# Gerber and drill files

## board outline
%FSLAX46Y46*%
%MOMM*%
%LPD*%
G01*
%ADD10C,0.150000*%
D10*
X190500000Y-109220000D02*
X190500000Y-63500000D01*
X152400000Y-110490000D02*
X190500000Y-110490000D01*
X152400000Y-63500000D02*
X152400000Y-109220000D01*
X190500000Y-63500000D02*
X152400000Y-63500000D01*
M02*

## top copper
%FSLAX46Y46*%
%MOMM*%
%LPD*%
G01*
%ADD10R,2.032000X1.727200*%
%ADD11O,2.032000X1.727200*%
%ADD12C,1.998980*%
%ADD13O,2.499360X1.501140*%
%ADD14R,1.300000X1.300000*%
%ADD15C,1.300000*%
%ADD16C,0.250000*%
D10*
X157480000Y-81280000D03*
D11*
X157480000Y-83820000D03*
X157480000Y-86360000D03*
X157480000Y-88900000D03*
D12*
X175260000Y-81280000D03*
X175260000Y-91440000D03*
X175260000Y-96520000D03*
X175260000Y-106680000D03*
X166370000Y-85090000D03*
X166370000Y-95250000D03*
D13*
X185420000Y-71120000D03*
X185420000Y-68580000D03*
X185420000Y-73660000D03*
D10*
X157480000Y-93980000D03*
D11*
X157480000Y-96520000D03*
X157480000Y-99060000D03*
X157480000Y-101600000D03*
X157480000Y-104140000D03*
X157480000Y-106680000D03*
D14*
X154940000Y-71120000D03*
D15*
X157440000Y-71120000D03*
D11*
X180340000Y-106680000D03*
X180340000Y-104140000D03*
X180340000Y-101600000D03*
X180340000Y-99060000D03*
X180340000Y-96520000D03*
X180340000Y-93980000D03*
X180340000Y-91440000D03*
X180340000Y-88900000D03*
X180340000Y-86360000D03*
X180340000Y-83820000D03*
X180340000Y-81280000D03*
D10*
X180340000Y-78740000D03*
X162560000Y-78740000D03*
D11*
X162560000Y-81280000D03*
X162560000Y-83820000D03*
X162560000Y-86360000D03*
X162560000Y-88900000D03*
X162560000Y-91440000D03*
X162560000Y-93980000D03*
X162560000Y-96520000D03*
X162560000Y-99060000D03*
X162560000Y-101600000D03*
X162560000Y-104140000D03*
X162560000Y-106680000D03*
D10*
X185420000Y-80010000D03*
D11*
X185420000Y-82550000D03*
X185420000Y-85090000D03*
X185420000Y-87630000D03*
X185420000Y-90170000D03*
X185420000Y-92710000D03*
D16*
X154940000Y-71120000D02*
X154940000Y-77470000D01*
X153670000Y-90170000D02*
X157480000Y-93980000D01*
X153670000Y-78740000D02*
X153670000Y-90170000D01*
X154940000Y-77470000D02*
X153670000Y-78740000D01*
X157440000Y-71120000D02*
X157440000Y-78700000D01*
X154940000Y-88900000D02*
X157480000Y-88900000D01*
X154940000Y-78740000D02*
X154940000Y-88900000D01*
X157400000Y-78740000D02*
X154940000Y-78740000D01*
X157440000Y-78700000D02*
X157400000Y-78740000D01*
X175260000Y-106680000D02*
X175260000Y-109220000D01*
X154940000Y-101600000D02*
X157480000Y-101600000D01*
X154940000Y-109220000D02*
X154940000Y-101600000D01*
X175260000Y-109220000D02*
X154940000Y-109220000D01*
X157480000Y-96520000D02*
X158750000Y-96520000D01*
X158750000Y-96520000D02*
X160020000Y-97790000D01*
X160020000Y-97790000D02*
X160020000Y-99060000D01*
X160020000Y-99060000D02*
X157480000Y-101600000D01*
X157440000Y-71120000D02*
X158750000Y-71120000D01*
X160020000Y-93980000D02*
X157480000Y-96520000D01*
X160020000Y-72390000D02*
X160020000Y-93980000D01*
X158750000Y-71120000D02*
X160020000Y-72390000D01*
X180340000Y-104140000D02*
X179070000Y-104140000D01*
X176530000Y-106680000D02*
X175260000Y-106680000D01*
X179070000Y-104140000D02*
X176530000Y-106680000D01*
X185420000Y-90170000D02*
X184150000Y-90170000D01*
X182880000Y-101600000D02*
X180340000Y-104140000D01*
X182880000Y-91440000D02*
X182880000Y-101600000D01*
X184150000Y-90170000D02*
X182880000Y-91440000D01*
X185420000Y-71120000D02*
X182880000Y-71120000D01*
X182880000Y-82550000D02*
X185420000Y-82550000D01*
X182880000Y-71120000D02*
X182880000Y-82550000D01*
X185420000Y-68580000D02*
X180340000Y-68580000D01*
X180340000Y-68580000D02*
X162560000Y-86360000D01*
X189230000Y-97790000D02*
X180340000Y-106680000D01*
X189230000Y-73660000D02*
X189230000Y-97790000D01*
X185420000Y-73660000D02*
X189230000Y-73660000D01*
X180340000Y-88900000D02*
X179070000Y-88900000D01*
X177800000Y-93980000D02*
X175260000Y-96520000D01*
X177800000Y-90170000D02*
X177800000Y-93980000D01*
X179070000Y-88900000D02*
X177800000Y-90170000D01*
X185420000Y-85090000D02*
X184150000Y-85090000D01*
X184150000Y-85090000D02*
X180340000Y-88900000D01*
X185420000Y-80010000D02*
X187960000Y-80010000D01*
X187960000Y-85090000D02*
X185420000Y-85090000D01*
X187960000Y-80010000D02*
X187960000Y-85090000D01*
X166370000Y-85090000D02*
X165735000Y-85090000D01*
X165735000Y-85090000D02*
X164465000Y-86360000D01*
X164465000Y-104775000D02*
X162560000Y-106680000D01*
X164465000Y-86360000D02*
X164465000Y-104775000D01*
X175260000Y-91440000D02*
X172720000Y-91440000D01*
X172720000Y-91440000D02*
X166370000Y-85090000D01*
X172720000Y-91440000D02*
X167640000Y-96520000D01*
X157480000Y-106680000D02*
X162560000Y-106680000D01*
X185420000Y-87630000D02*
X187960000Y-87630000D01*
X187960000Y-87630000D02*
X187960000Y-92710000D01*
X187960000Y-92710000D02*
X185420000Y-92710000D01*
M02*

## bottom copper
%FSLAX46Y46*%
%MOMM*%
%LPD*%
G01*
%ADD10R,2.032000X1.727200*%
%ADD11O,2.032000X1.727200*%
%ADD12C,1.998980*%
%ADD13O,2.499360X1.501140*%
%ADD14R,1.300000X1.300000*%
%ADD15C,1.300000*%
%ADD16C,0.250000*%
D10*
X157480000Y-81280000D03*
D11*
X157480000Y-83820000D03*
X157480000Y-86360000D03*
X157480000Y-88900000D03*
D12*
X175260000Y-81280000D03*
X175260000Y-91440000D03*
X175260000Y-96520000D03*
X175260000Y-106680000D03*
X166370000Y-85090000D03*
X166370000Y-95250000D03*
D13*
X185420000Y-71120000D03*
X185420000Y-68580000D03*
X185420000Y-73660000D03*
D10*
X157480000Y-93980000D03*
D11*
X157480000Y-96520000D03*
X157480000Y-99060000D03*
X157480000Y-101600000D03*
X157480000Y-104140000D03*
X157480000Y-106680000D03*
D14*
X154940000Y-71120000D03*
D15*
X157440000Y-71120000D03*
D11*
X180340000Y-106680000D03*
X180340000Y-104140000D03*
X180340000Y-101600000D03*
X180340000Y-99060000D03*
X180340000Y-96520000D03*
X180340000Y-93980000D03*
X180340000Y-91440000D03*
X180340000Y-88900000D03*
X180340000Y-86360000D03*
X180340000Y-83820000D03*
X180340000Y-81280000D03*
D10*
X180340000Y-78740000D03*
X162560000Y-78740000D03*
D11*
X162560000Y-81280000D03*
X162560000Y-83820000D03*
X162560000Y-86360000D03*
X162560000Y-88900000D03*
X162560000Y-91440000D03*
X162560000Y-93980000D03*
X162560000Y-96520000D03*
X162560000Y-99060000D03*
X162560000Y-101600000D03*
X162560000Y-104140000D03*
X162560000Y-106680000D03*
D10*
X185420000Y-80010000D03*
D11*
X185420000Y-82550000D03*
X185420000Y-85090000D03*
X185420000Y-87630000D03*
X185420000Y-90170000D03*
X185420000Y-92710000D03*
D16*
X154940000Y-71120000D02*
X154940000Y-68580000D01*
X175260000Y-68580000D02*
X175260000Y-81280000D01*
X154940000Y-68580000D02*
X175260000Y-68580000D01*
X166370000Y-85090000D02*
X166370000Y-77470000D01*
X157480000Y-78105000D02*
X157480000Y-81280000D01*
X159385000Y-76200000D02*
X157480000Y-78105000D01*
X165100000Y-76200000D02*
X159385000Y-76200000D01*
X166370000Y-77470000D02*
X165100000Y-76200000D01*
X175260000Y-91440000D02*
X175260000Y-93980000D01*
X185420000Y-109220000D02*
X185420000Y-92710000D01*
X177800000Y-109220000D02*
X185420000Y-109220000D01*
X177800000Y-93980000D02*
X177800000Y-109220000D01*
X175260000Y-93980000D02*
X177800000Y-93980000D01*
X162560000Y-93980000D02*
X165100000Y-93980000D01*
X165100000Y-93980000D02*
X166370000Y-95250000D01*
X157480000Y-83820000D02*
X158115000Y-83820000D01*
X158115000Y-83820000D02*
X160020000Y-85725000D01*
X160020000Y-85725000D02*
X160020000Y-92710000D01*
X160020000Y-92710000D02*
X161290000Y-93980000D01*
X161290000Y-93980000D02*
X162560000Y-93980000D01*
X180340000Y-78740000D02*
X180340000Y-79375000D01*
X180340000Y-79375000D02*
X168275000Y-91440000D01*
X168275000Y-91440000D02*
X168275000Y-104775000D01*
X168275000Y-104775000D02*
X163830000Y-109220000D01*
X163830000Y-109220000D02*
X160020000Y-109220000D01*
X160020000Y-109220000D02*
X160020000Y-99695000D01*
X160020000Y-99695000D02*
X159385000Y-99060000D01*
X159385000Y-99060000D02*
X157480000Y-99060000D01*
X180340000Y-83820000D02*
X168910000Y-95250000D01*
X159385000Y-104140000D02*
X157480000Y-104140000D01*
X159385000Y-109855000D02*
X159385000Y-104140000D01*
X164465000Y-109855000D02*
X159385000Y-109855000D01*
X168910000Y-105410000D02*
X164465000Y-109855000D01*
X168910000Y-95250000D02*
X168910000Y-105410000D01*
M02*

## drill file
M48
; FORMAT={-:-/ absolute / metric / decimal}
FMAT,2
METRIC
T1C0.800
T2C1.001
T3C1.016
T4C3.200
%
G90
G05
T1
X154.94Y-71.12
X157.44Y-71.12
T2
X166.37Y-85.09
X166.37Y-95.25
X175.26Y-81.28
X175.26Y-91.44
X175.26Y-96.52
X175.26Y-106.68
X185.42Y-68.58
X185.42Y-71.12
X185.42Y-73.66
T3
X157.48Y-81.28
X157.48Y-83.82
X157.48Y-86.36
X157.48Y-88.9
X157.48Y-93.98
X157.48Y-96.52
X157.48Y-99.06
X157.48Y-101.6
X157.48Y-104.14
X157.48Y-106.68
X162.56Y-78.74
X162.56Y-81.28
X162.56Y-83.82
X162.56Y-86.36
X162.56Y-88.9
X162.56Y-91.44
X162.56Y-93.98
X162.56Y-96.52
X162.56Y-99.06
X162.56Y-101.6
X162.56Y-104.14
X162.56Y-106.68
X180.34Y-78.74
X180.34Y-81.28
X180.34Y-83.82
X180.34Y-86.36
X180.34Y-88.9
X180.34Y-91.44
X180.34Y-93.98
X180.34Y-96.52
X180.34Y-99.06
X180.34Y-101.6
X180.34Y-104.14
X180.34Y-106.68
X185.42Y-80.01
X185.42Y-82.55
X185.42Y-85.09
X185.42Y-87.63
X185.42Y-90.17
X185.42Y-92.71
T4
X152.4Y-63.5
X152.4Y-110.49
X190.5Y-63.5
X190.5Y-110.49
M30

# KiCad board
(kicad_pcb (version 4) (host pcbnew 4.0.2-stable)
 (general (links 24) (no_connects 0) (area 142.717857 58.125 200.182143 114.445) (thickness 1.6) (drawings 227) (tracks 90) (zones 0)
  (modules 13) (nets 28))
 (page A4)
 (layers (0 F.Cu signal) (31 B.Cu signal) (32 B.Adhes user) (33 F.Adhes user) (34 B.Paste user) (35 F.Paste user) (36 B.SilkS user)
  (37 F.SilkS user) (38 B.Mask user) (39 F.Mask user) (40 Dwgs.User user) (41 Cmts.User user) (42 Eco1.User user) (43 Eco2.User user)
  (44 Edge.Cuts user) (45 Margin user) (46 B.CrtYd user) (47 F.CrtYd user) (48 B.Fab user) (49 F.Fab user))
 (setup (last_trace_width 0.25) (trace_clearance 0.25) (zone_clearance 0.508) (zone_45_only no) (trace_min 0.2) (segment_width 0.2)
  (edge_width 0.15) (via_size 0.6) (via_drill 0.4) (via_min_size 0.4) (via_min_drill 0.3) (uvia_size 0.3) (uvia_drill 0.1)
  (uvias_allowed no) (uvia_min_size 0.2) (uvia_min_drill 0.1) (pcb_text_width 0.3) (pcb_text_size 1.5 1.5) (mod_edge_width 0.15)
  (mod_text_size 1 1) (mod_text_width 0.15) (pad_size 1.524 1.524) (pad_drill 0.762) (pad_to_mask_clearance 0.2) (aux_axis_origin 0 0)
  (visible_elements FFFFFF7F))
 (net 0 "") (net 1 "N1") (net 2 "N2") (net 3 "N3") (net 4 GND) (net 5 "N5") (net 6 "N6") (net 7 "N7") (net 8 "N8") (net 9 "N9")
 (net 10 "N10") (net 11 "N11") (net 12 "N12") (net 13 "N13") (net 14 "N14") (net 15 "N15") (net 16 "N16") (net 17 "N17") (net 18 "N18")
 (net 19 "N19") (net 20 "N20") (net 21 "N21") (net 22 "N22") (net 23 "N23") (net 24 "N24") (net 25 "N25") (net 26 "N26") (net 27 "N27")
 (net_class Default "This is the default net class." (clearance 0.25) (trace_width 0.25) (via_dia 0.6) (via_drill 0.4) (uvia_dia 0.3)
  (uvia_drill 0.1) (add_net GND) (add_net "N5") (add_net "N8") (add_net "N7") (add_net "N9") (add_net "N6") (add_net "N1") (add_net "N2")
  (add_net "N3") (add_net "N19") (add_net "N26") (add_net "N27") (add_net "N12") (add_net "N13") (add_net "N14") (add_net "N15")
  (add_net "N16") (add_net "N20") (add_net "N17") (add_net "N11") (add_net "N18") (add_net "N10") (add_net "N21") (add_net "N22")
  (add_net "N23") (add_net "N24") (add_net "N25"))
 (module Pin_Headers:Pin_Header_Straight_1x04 (layer F.Cu) (at 157.48 81.28)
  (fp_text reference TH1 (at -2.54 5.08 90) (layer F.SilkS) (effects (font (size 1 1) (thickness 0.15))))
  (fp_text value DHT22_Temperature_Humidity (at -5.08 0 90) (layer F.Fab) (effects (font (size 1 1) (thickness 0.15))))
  (pad 1 thru_hole rect (at 0 0) (size 2.032 1.7272) (drill 1.016) (layers *.Cu *.Mask F.SilkS) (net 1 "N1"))
  (pad 2 thru_hole oval (at 0 2.54) (size 2.032 1.7272) (drill 1.016) (layers *.Cu *.Mask F.SilkS) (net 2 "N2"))
  (pad 3 thru_hole oval (at 0 5.08) (size 2.032 1.7272) (drill 1.016) (layers *.Cu *.Mask F.SilkS) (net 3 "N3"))
  (pad 4 thru_hole oval (at 0 7.62) (size 2.032 1.7272) (drill 1.016) (layers *.Cu *.Mask F.SilkS) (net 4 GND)))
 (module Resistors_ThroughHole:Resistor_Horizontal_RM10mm (layer F.Cu) (at 175.26 81.28 270)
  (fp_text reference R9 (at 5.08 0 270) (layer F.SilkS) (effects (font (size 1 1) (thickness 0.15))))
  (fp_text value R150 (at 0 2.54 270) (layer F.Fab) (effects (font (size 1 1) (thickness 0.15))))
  (pad 1 thru_hole circle (at 0 0 270) (size 1.99898 1.99898) (drill 1.00076) (layers *.Cu *.SilkS *.Mask) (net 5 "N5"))
  (pad 2 thru_hole circle (at 10.16 0 270) (size 1.99898 1.99898) (drill 1.00076) (layers *.Cu *.SilkS *.Mask) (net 1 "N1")))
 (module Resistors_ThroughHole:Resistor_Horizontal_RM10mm (layer F.Cu) (at 175.26 96.52 270)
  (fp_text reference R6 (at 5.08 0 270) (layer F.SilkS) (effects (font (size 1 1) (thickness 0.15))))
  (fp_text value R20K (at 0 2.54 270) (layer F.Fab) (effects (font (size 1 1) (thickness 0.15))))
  (pad 1 thru_hole circle (at 0 0 270) (size 1.99898 1.99898) (drill 1.00076) (layers *.Cu *.SilkS *.Mask) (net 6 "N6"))
  (pad 2 thru_hole circle (at 10.16 0 270) (size 1.99898 1.99898) (drill 1.00076) (layers *.Cu *.SilkS *.Mask) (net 4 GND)))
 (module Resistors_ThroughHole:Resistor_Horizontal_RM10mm (layer F.Cu) (at 166.37 85.09 270)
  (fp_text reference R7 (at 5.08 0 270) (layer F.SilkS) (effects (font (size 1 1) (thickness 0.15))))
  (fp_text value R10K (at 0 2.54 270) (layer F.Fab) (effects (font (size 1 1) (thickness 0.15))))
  (pad 1 thru_hole circle (at 0 0 270) (size 1.99898 1.99898) (drill 1.00076) (layers *.Cu *.SilkS *.Mask) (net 1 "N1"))
  (pad 2 thru_hole circle (at 10.16 0 270) (size 1.99898 1.99898) (drill 1.00076) (layers *.Cu *.SilkS *.Mask) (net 2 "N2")))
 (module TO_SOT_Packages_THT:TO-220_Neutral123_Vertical (layer F.Cu) (at 185.42 71.12 270)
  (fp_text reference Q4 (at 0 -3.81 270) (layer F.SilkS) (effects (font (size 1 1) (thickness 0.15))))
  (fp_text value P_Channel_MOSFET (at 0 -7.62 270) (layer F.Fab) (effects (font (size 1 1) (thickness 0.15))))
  (pad 2 thru_hole oval (at 0 0) (size 2.49936 1.50114) (drill 1.00076) (layers *.Cu *.Mask F.SilkS) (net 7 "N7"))
  (pad 1 thru_hole oval (at -2.54 0) (size 2.49936 1.50114) (drill 1.00076) (layers *.Cu *.Mask F.SilkS) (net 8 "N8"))
  (pad 3 thru_hole oval (at 2.54 0) (size 2.49936 1.50114) (drill 1.00076) (layers *.Cu *.Mask F.SilkS) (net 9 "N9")))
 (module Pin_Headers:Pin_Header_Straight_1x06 (layer F.Cu) (at 157.48 93.98)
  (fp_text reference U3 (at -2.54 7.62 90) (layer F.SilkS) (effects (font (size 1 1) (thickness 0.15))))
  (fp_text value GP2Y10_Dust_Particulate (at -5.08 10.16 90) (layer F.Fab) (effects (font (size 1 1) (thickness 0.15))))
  (pad 1 thru_hole rect (at 0 0) (size 2.032 1.7272) (drill 1.016) (layers *.Cu *.Mask F.SilkS) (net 5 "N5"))
  (pad 2 thru_hole oval (at 0 2.54) (size 2.032 1.7272) (drill 1.016) (layers *.Cu *.Mask F.SilkS) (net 4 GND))
  (pad 3 thru_hole oval (at 0 5.08) (size 2.032 1.7272) (drill 1.016) (layers *.Cu *.Mask F.SilkS) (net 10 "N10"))
  (pad 4 thru_hole oval (at 0 7.62) (size 2.032 1.7272) (drill 1.016) (layers *.Cu *.Mask F.SilkS) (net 4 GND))
  (pad 5 thru_hole oval (at 0 10.16) (size 2.032 1.7272) (drill 1.016) (layers *.Cu *.Mask F.SilkS) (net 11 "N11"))
  (pad 6 thru_hole oval (at 0 12.7) (size 2.032 1.7272) (drill 1.016) (layers *.Cu *.Mask F.SilkS) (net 1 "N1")))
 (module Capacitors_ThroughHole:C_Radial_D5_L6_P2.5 (layer F.Cu) (at 154.94 71.12)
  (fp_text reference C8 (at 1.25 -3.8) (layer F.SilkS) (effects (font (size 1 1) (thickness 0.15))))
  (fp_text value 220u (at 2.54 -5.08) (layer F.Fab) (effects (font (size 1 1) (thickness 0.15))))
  (pad 1 thru_hole rect (at 0 0) (size 1.3 1.3) (drill 0.8) (layers *.Cu *.Mask F.SilkS) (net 5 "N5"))
  (pad 2 thru_hole circle (at 2.5 0) (size 1.3 1.3) (drill 0.8) (layers *.Cu *.Mask F.SilkS) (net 4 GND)))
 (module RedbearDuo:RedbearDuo (layer F.Cu) (at 162.56 78.74)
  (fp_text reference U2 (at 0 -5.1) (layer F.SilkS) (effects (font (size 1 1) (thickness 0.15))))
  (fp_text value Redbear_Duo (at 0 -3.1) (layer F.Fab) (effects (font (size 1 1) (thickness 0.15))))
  (pad 13 thru_hole oval (at 17.78 27.94) (size 2.032 1.7272) (drill 1.016) (layers *.Cu *.Mask F.SilkS) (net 9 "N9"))
  (pad 14 thru_hole oval (at 17.78 25.4) (size 2.032 1.7272) (drill 1.016) (layers *.Cu *.Mask F.SilkS) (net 4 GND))
  (pad 15 thru_hole oval (at 17.78 22.86) (size 2.032 1.7272) (drill 1.016) (layers *.Cu *.Mask F.SilkS) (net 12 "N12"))
  (pad 16 thru_hole oval (at 17.78 20.32) (size 2.032 1.7272) (drill 1.016) (layers *.Cu *.Mask F.SilkS) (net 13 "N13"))
  (pad 17 thru_hole oval (at 17.78 17.78) (size 2.032 1.7272) (drill 1.016) (layers *.Cu *.Mask F.SilkS) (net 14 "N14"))
  (pad 18 thru_hole oval (at 17.78 15.24) (size 2.032 1.7272) (drill 1.016) (layers *.Cu *.Mask F.SilkS) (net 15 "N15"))
  (pad 19 thru_hole oval (at 17.78 12.7) (size 2.032 1.7272) (drill 1.016) (layers *.Cu *.Mask F.SilkS) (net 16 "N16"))
  (pad 20 thru_hole oval (at 17.78 10.16) (size 2.032 1.7272) (drill 1.016) (layers *.Cu *.Mask F.SilkS) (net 6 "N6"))
  (pad 21 thru_hole oval (at 17.78 7.62) (size 2.032 1.7272) (drill 1.016) (layers *.Cu *.Mask F.SilkS) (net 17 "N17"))
  (pad 22 thru_hole oval (at 17.78 5.08) (size 2.032 1.7272) (drill 1.016) (layers *.Cu *.Mask F.SilkS) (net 11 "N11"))
  (pad 23 thru_hole oval (at 17.78 2.54) (size 2.032 1.7272) (drill 1.016) (layers *.Cu *.Mask F.SilkS) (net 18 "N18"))
  (pad 24 thru_hole rect (at 17.78 0) (size 2.032 1.7272) (drill 1.016) (layers *.Cu *.Mask F.SilkS) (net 10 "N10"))
  (pad 1 thru_hole rect (at 0 0) (size 2.032 1.7272) (drill 1.016) (layers *.Cu *.Mask F.SilkS) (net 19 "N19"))
  (pad 2 thru_hole oval (at 0 2.54) (size 2.032 1.7272) (drill 1.016) (layers *.Cu *.Mask F.SilkS) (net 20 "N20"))
  (pad 3 thru_hole oval (at 0 5.08) (size 2.032 1.7272) (drill 1.016) (layers *.Cu *.Mask F.SilkS) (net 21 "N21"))
  (pad 4 thru_hole oval (at 0 7.62) (size 2.032 1.7272) (drill 1.016) (layers *.Cu *.Mask F.SilkS) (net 8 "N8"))
  (pad 5 thru_hole oval (at 0 10.16) (size 2.032 1.7272) (drill 1.016) (layers *.Cu *.Mask F.SilkS) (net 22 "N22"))
  (pad 6 thru_hole oval (at 0 12.7) (size 2.032 1.7272) (drill 1.016) (layers *.Cu *.Mask F.SilkS) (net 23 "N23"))
  (pad 7 thru_hole oval (at 0 15.24) (size 2.032 1.7272) (drill 1.016) (layers *.Cu *.Mask F.SilkS) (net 2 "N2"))
  (pad 8 thru_hole oval (at 0 17.78) (size 2.032 1.7272) (drill 1.016) (layers *.Cu *.Mask F.SilkS) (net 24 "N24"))
  (pad 9 thru_hole oval (at 0 20.32) (size 2.032 1.7272) (drill 1.016) (layers *.Cu *.Mask F.SilkS) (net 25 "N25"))
  (pad 10 thru_hole oval (at 0 22.86) (size 2.032 1.7272) (drill 1.016) (layers *.Cu *.Mask F.SilkS) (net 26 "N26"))
  (pad 11 thru_hole oval (at 0 25.4) (size 2.032 1.7272) (drill 1.016) (layers *.Cu *.Mask F.SilkS) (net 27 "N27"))
  (pad 12 thru_hole oval (at 0 27.94) (size 2.032 1.7272) (drill 1.016) (layers *.Cu *.Mask F.SilkS) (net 1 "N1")))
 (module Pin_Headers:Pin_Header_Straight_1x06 (layer F.Cu) (at 185.42 80.01)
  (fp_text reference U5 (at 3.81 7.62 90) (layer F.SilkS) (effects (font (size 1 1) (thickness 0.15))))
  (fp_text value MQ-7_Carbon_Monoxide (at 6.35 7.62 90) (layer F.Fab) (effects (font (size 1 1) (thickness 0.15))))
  (pad 1 thru_hole rect (at 0 0) (size 2.032 1.7272) (drill 1.016) (layers *.Cu *.Mask F.SilkS) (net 6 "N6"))
  (pad 2 thru_hole oval (at 0 2.54) (size 2.032 1.7272) (drill 1.016) (layers *.Cu *.Mask F.SilkS) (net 7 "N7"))
  (pad 3 thru_hole oval (at 0 5.08) (size 2.032 1.7272) (drill 1.016) (layers *.Cu *.Mask F.SilkS) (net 6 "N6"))
  (pad 4 thru_hole oval (at 0 7.62) (size 2.032 1.7272) (drill 1.016) (layers *.Cu *.Mask F.SilkS) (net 1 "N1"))
  (pad 5 thru_hole oval (at 0 10.16) (size 2.032 1.7272) (drill 1.016) (layers *.Cu *.Mask F.SilkS) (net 4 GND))
  (pad 6 thru_hole oval (at 0 12.7) (size 2.032 1.7272) (drill 1.016) (layers *.Cu *.Mask F.SilkS) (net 1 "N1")))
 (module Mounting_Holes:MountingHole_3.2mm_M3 (layer F.Cu) (at 190.5 63.5)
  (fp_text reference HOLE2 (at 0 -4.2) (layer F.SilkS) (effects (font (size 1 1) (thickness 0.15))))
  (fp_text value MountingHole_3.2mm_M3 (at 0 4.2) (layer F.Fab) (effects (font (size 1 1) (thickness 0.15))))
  (pad 1 np_thru_hole circle (at 0 0) (size 3.2 3.2) (drill 3.2) (layers *.Cu *.Mask F.SilkS)))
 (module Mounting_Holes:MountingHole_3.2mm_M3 (layer F.Cu) (at 190.5 110.49)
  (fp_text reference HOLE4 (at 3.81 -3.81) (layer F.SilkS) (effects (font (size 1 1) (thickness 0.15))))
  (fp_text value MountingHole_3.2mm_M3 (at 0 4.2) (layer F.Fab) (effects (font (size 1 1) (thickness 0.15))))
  (pad 1 np_thru_hole circle (at 0 0) (size 3.2 3.2) (drill 3.2) (layers *.Cu *.Mask F.SilkS)))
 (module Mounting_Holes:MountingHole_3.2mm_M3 (layer F.Cu) (at 152.4 63.5)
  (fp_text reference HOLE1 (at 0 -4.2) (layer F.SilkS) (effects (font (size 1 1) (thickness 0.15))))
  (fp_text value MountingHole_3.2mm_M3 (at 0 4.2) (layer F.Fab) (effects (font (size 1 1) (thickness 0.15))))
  (pad 1 np_thru_hole circle (at 0 0) (size 3.2 3.2) (drill 3.2) (layers *.Cu *.Mask F.SilkS)))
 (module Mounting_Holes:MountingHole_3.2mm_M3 (layer F.Cu) (at 152.4 110.49)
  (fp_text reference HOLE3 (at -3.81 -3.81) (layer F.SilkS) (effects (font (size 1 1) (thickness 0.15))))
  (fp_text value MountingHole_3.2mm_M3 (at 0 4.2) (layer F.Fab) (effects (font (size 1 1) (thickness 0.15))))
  (pad 1 np_thru_hole circle (at 0 0) (size 3.2 3.2) (drill 3.2) (layers *.Cu *.Mask F.SilkS)))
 (gr_line (start 190.5 109.22) (end 190.5 63.5) (angle 90) (layer Edge.Cuts) (width 0.15))
 (gr_line (start 152.4 110.49) (end 190.5 110.49) (angle 90) (layer Edge.Cuts) (width 0.15))
 (gr_line (start 152.4 63.5) (end 152.4 109.22) (angle 90) (layer Edge.Cuts) (width 0.15))
 (gr_line (start 190.5 63.5) (end 152.4 63.5) (angle 90) (layer Edge.Cuts) (width 0.15))
 (segment (start 154.94 71.12) (end 154.94 68.58) (width 0.25) (layer B.Cu) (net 5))
 (segment (start 175.26 68.58) (end 175.26 81.28) (width 0.25) (layer B.Cu) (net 5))
 (segment (start 154.94 68.58) (end 175.26 68.58) (width 0.25) (layer B.Cu) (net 5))
 (segment (start 154.94 71.12) (end 154.94 77.47) (width 0.25) (layer F.Cu) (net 5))
 (segment (start 153.67 90.17) (end 157.48 93.98) (width 0.25) (layer F.Cu) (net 5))
 (segment (start 153.67 78.74) (end 153.67 90.17) (width 0.25) (layer F.Cu) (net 5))
 (segment (start 154.94 77.47) (end 153.67 78.74) (width 0.25) (layer F.Cu) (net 5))
 (segment (start 157.44 71.12) (end 157.44 78.7) (width 0.25) (layer F.Cu) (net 4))
 (segment (start 154.94 88.9) (end 157.48 88.9) (width 0.25) (layer F.Cu) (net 4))
 (segment (start 154.94 78.74) (end 154.94 88.9) (width 0.25) (layer F.Cu) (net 4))
 (segment (start 157.4 78.74) (end 154.94 78.74) (width 0.25) (layer F.Cu) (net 4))
 (segment (start 157.44 78.7) (end 157.4 78.74) (width 0.25) (layer F.Cu) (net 4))
 (segment (start 175.26 106.68) (end 175.26 109.22) (width 0.25) (layer F.Cu) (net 4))
 (segment (start 154.94 101.6) (end 157.48 101.6) (width 0.25) (layer F.Cu) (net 4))
 (segment (start 154.94 109.22) (end 154.94 101.6) (width 0.25) (layer F.Cu) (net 4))
 (segment (start 175.26 109.22) (end 154.94 109.22) (width 0.25) (layer F.Cu) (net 4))
 (segment (start 157.48 96.52) (end 158.75 96.52) (width 0.25) (layer F.Cu) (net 4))
 (segment (start 158.75 96.52) (end 160.02 97.79) (width 0.25) (layer F.Cu) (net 4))
 (segment (start 160.02 97.79) (end 160.02 99.06) (width 0.25) (layer F.Cu) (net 4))
 (segment (start 160.02 99.06) (end 157.48 101.6) (width 0.25) (layer F.Cu) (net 4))
 (segment (start 157.44 71.12) (end 158.75 71.12) (width 0.25) (layer F.Cu) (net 4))
 (segment (start 160.02 93.98) (end 157.48 96.52) (width 0.25) (layer F.Cu) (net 4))
 (segment (start 160.02 72.39) (end 160.02 93.98) (width 0.25) (layer F.Cu) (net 4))
 (segment (start 158.75 71.12) (end 160.02 72.39) (width 0.25) (layer F.Cu) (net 4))
 (segment (start 180.34 104.14) (end 179.07 104.14) (width 0.25) (layer F.Cu) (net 4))
 (segment (start 176.53 106.68) (end 175.26 106.68) (width 0.25) (layer F.Cu) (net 4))
 (segment (start 179.07 104.14) (end 176.53 106.68) (width 0.25) (layer F.Cu) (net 4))
 (segment (start 185.42 90.17) (end 184.15 90.17) (width 0.25) (layer F.Cu) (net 4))
 (segment (start 182.88 101.6) (end 180.34 104.14) (width 0.25) (layer F.Cu) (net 4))
 (segment (start 182.88 91.44) (end 182.88 101.6) (width 0.25) (layer F.Cu) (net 4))
 (segment (start 184.15 90.17) (end 182.88 91.44) (width 0.25) (layer F.Cu) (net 4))
 (segment (start 185.42 71.12) (end 182.88 71.12) (width 0.25) (layer F.Cu) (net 7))
 (segment (start 182.88 82.55) (end 185.42 82.55) (width 0.25) (layer F.Cu) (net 7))
 (segment (start 182.88 71.12) (end 182.88 82.55) (width 0.25) (layer F.Cu) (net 7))
 (segment (start 185.42 68.58) (end 180.34 68.58) (width 0.25) (layer F.Cu) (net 8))
 (segment (start 180.34 68.58) (end 162.56 86.36) (width 0.25) (layer F.Cu) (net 8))
 (segment (start 189.23 97.79) (end 180.34 106.68) (width 0.25) (layer F.Cu) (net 9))
 (segment (start 189.23 73.66) (end 189.23 97.79) (width 0.25) (layer F.Cu) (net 9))
 (segment (start 185.42 73.66) (end 189.23 73.66) (width 0.25) (layer F.Cu) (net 9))
 (segment (start 180.34 88.9) (end 179.07 88.9) (width 0.25) (layer F.Cu) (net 6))
 (segment (start 177.8 93.98) (end 175.26 96.52) (width 0.25) (layer F.Cu) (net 6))
 (segment (start 177.8 90.17) (end 177.8 93.98) (width 0.25) (layer F.Cu) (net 6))
 (segment (start 179.07 88.9) (end 177.8 90.17) (width 0.25) (layer F.Cu) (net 6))
 (segment (start 185.42 85.09) (end 184.15 85.09) (width 0.25) (layer F.Cu) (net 6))
 (segment (start 184.15 85.09) (end 180.34 88.9) (width 0.25) (layer F.Cu) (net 6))
 (segment (start 185.42 80.01) (end 187.96 80.01) (width 0.25) (layer F.Cu) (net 6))
 (segment (start 187.96 85.09) (end 185.42 85.09) (width 0.25) (layer F.Cu) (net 6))
 (segment (start 187.96 80.01) (end 187.96 85.09) (width 0.25) (layer F.Cu) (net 6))
 (segment (start 166.37 85.09) (end 166.37 77.47) (width 0.25) (layer B.Cu) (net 1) (status 400000))
 (segment (start 157.48 78.105) (end 157.48 81.28) (width 0.25) (layer B.Cu) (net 1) (status 800000))
 (segment (start 159.385 76.2) (end 157.48 78.105) (width 0.25) (layer B.Cu) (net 1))
 (segment (start 165.1 76.2) (end 159.385 76.2) (width 0.25) (layer B.Cu) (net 1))
 (segment (start 166.37 77.47) (end 165.1 76.2) (width 0.25) (layer B.Cu) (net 1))
 (segment (start 166.37 85.09) (end 165.735 85.09) (width 0.25) (layer F.Cu) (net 1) (status C00000))
 (segment (start 165.735 85.09) (end 164.465 86.36) (width 0.25) (layer F.Cu) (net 1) (status 400000))
 (segment (start 164.465 104.775) (end 162.56 106.68) (width 0.25) (layer F.Cu) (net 1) (status 800000))
 (segment (start 164.465 86.36) (end 164.465 104.775) (width 0.25) (layer F.Cu) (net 1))
 (segment (start 175.26 91.44) (end 172.72 91.44) (width 0.25) (layer F.Cu) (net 1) (status 400000))
 (segment (start 172.72 91.44) (end 166.37 85.09) (width 0.25) (layer F.Cu) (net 1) (status 800000))
 (segment (start 175.26 91.44) (end 175.26 93.98) (width 0.25) (layer B.Cu) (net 1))
 (segment (start 185.42 109.22) (end 185.42 92.71) (width 0.25) (layer B.Cu) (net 1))
 (segment (start 177.8 109.22) (end 185.42 109.22) (width 0.25) (layer B.Cu) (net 1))
 (segment (start 177.8 93.98) (end 177.8 109.22) (width 0.25) (layer B.Cu) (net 1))
 (segment (start 175.26 93.98) (end 177.8 93.98) (width 0.25) (layer B.Cu) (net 1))
 (segment (start 172.72 91.44) (end 167.64 96.52) (width 0.25) (layer F.Cu) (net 1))
 (segment (start 157.48 106.68) (end 162.56 106.68) (width 0.25) (layer F.Cu) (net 1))
 (segment (start 185.42 87.63) (end 187.96 87.63) (width 0.25) (layer F.Cu) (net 1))
 (segment (start 187.96 87.63) (end 187.96 92.71) (width 0.25) (layer F.Cu) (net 1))
 (segment (start 187.96 92.71) (end 185.42 92.71) (width 0.25) (layer F.Cu) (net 1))
 (segment (start 162.56 93.98) (end 165.1 93.98) (width 0.25) (layer B.Cu) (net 2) (status 400000))
 (segment (start 165.1 93.98) (end 166.37 95.25) (width 0.25) (layer B.Cu) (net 2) (status 800000))
 (segment (start 157.48 83.82) (end 158.115 83.82) (width 0.25) (layer B.Cu) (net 2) (status C00000))
 (segment (start 158.115 83.82) (end 160.02 85.725) (width 0.25) (layer B.Cu) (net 2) (status 400000))
 (segment (start 160.02 85.725) (end 160.02 92.71) (width 0.25) (layer B.Cu) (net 2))
 (segment (start 160.02 92.71) (end 161.29 93.98) (width 0.25) (layer B.Cu) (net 2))
 (segment (start 161.29 93.98) (end 162.56 93.98) (width 0.25) (layer B.Cu) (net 2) (status 800000))
 (segment (start 180.34 78.74) (end 180.34 79.375) (width 0.25) (layer B.Cu) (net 10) (status C00000))
 (segment (start 180.34 79.375) (end 168.275 91.44) (width 0.25) (layer B.Cu) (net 10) (status 400000))
 (segment (start 168.275 91.44) (end 168.275 104.775) (width 0.25) (layer B.Cu) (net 10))
 (segment (start 168.275 104.775) (end 163.83 109.22) (width 0.25) (layer B.Cu) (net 10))
 (segment (start 163.83 109.22) (end 160.02 109.22) (width 0.25) (layer B.Cu) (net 10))
 (segment (start 160.02 109.22) (end 160.02 99.695) (width 0.25) (layer B.Cu) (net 10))
 (segment (start 160.02 99.695) (end 159.385 99.06) (width 0.25) (layer B.Cu) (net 10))
 (segment (start 159.385 99.06) (end 157.48 99.06) (width 0.25) (layer B.Cu) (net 10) (status 800000))
 (segment (start 180.34 83.82) (end 168.91 95.25) (width 0.25) (layer B.Cu) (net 11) (status 400000))
 (segment (start 159.385 104.14) (end 157.48 104.14) (width 0.25) (layer B.Cu) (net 11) (status 800000))
 (segment (start 159.385 109.855) (end 159.385 104.14) (width 0.25) (layer B.Cu) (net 11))
 (segment (start 164.465 109.855) (end 159.385 109.855) (width 0.25) (layer B.Cu) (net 11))
 (segment (start 168.91 105.41) (end 164.465 109.855) (width 0.25) (layer B.Cu) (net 11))
 (segment (start 168.91 95.25) (end 168.91 105.41) (width 0.25) (layer B.Cu) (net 11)))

